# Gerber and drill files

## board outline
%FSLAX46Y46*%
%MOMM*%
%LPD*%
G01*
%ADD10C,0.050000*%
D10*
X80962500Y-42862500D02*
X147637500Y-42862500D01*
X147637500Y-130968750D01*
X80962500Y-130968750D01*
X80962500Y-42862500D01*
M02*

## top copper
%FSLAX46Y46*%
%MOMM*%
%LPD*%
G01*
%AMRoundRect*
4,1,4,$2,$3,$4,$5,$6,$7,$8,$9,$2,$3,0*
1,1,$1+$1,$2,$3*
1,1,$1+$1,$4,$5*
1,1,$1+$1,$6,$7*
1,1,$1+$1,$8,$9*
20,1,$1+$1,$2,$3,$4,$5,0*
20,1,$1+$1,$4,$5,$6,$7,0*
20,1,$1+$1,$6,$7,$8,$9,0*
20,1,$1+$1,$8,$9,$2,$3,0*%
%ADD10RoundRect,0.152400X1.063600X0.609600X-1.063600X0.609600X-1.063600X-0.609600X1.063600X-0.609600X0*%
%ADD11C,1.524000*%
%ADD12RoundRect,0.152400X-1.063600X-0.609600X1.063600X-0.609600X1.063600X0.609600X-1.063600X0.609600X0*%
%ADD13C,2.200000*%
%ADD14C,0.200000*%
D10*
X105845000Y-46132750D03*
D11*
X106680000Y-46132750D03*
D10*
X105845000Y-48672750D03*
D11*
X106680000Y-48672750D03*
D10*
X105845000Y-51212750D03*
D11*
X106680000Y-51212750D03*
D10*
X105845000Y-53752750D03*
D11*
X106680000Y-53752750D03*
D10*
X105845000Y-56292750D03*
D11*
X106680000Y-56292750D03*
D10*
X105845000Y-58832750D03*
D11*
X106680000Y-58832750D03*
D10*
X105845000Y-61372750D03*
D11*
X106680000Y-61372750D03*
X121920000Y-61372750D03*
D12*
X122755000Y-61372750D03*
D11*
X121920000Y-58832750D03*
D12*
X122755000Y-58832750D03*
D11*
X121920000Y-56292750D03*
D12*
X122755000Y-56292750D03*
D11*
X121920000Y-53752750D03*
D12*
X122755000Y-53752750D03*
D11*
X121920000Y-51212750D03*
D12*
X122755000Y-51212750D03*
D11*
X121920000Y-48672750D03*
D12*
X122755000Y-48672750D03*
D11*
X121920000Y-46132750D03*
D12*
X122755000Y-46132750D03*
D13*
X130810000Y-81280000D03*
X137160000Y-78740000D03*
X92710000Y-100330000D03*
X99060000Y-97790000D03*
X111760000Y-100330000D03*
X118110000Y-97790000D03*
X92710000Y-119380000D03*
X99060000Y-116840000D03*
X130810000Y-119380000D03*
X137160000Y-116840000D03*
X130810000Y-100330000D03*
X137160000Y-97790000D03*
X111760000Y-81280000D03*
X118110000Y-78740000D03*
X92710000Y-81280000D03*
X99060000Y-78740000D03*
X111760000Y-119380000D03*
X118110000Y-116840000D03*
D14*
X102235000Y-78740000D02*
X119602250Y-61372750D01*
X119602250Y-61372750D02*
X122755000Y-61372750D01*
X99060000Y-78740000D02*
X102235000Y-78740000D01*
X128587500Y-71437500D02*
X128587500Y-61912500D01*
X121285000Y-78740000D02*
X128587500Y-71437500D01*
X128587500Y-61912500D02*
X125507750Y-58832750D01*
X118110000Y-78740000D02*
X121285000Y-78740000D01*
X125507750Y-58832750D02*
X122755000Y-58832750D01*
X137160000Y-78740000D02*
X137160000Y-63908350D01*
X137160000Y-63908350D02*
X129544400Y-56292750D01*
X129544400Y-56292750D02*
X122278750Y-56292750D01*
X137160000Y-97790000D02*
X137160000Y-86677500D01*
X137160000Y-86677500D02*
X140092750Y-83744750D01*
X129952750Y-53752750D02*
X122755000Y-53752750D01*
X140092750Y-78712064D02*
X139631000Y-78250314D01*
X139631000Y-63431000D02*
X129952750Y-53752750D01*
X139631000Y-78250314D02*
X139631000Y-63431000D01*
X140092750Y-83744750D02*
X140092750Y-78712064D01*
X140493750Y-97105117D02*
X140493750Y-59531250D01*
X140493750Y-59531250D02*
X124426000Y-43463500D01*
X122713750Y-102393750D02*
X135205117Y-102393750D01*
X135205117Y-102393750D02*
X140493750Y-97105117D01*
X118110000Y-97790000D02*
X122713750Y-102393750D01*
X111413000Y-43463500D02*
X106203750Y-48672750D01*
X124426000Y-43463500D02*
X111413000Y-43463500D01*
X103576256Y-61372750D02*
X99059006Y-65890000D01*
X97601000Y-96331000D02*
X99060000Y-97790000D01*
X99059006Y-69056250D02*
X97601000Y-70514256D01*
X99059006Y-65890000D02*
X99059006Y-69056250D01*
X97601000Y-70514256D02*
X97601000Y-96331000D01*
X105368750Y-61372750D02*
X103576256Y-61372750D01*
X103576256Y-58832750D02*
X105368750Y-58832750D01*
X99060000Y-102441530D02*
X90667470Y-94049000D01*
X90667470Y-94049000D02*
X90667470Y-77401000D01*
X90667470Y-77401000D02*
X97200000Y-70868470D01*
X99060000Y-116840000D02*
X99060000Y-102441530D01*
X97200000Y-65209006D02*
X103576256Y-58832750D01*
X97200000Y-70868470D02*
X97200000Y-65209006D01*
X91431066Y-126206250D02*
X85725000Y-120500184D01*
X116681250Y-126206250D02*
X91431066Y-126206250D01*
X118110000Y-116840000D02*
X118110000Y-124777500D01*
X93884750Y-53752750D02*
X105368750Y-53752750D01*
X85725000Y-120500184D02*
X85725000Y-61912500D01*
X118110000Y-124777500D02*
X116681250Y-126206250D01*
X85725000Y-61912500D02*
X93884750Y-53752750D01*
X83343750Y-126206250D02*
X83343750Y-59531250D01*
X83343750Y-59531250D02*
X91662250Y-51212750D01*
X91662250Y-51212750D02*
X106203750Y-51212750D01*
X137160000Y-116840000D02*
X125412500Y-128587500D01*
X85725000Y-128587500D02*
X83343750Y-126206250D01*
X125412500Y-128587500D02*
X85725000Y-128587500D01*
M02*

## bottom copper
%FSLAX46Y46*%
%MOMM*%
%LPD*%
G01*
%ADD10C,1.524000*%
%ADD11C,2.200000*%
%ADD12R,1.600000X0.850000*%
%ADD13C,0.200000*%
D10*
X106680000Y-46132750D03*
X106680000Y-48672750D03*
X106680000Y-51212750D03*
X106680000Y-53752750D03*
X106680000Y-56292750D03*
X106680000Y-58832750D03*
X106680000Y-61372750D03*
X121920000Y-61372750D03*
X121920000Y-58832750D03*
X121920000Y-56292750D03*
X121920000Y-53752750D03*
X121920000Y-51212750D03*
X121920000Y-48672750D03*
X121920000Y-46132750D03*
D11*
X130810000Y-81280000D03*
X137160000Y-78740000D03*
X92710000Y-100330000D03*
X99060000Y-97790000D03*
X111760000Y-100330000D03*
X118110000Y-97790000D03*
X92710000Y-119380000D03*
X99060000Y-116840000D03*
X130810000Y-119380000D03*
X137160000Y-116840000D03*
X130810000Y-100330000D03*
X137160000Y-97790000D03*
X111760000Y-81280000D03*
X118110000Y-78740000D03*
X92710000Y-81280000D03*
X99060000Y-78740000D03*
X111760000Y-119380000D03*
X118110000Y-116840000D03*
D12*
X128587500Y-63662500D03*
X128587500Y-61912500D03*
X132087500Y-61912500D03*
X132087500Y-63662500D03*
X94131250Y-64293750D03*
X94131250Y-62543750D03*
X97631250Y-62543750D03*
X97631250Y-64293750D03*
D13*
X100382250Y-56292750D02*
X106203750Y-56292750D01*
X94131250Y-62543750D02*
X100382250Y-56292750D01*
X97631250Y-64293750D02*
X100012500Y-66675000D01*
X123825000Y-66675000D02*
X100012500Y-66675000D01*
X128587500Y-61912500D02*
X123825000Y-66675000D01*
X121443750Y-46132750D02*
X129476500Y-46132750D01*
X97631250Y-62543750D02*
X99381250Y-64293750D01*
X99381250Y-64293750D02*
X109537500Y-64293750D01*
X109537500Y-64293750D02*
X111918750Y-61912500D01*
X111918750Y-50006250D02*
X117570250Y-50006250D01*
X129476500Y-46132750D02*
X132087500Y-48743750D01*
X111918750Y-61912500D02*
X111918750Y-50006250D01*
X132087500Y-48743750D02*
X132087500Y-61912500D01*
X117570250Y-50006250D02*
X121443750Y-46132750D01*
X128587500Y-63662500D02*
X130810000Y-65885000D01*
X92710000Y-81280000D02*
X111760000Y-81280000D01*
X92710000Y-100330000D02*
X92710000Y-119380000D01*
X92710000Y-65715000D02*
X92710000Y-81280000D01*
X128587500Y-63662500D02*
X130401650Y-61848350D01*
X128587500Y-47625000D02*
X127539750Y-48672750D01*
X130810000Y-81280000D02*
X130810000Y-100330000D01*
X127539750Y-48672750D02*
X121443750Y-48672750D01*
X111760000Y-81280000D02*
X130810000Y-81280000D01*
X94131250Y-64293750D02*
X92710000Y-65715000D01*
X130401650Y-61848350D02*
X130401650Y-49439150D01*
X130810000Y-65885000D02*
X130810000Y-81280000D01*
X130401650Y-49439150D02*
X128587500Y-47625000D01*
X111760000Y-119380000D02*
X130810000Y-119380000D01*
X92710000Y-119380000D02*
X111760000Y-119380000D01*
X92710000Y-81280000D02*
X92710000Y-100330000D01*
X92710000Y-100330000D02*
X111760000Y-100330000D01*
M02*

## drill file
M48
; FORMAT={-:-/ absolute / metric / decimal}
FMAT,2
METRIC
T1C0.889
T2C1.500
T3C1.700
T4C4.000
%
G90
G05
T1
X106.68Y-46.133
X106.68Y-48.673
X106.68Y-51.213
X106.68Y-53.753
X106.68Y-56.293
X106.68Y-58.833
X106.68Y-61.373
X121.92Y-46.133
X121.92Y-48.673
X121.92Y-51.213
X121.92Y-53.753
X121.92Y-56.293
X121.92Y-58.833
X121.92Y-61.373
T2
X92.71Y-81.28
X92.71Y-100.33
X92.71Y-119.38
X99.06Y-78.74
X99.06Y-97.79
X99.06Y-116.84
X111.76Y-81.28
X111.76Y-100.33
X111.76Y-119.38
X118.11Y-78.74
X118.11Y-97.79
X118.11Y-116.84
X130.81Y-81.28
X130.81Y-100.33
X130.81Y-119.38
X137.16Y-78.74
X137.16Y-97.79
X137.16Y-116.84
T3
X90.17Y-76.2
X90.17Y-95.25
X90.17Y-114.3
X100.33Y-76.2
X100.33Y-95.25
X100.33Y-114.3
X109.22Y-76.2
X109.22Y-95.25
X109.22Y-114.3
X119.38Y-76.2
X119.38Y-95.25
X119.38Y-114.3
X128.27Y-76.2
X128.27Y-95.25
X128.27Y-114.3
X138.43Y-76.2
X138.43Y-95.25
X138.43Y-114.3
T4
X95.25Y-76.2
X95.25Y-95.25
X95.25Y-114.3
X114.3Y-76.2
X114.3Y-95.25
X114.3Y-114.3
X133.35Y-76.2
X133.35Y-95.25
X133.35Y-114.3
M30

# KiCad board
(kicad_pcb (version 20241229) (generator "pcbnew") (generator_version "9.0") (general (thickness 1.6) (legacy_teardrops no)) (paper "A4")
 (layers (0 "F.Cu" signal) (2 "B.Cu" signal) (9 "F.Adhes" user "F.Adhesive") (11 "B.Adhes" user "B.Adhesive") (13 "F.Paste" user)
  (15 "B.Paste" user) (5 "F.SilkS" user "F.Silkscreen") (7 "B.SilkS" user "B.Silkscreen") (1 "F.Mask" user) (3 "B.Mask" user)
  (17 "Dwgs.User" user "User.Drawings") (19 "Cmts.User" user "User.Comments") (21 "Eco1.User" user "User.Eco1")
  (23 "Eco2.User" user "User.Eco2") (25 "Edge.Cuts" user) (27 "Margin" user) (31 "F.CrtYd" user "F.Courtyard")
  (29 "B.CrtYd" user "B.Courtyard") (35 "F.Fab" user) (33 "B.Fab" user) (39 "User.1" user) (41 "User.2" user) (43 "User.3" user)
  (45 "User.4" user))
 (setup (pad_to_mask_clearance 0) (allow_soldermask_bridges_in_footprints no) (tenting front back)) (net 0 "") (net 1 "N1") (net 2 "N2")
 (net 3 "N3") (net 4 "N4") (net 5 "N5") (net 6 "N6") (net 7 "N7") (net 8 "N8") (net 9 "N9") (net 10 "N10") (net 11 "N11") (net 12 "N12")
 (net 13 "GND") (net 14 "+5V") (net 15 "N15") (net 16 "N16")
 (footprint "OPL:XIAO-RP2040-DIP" (layer "F.Cu") (at 114.3 53.75275)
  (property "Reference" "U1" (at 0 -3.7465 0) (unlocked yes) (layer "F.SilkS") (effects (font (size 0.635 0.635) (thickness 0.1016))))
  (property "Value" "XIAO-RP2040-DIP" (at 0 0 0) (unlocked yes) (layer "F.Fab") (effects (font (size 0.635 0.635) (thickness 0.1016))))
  (pad "1" smd roundrect (at -8.455 -7.62 180) (size 2.432 1.524) (layers "F.Cu" "F.Mask") (roundrect_rratio 0.1) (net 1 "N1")
   (thermal_bridge_angle 45))
  (pad "1" thru_hole circle (at -7.62 -7.62 180) (size 1.524 1.524) (drill 0.889) (layers "*.Cu" "*.Mask") (remove_unused_layers no)
   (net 1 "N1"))
  (pad "2" smd roundrect (at -8.455 -5.08 180) (size 2.432 1.524) (layers "F.Cu" "F.Mask") (roundrect_rratio 0.1) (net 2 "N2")
   (thermal_bridge_angle 45))
  (pad "2" thru_hole circle (at -7.62 -5.08 180) (size 1.524 1.524) (drill 0.889) (layers "*.Cu" "*.Mask") (remove_unused_layers no)
   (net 2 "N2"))
  (pad "3" smd roundrect (at -8.455 -2.54 180) (size 2.432 1.524) (layers "F.Cu" "F.Mask") (roundrect_rratio 0.1) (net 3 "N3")
   (thermal_bridge_angle 45))
  (pad "3" thru_hole circle (at -7.62 -2.54 180) (size 1.524 1.524) (drill 0.889) (layers "*.Cu" "*.Mask") (remove_unused_layers no)
   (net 3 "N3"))
  (pad "4" smd roundrect (at -8.455 0 180) (size 2.432 1.524) (layers "F.Cu" "F.Mask") (roundrect_rratio 0.1) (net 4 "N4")
   (thermal_bridge_angle 45))
  (pad "4" thru_hole circle (at -7.62 0 180) (size 1.524 1.524) (drill 0.889) (layers "*.Cu" "*.Mask") (remove_unused_layers no)
   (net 4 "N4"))
  (pad "5" smd roundrect (at -8.455 2.54 180) (size 2.432 1.524) (layers "F.Cu" "F.Mask") (roundrect_rratio 0.1) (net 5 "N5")
   (thermal_bridge_angle 45))
  (pad "5" thru_hole circle (at -7.62 2.54 180) (size 1.524 1.524) (drill 0.889) (layers "*.Cu" "*.Mask") (remove_unused_layers no)
   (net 5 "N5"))
  (pad "6" smd roundrect (at -8.455 5.08 180) (size 2.432 1.524) (layers "F.Cu" "F.Mask") (roundrect_rratio 0.1) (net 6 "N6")
   (thermal_bridge_angle 45))
  (pad "6" thru_hole circle (at -7.62 5.08 180) (size 1.524 1.524) (drill 0.889) (layers "*.Cu" "*.Mask") (remove_unused_layers no)
   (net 6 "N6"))
  (pad "7" smd roundrect (at -8.455 7.62 180) (size 2.432 1.524) (layers "F.Cu" "F.Mask") (roundrect_rratio 0.1) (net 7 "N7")
   (thermal_bridge_angle 45))
  (pad "7" thru_hole circle (at -7.62 7.62 180) (size 1.524 1.524) (drill 0.889) (layers "*.Cu" "*.Mask") (remove_unused_layers no)
   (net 7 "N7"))
  (pad "8" thru_hole circle (at 7.62 7.62) (size 1.524 1.524) (drill 0.889) (layers "*.Cu" "*.Mask") (remove_unused_layers no) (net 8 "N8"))
  (pad "8" smd roundrect (at 8.455 7.62) (size 2.432 1.524) (layers "F.Cu" "F.Mask") (roundrect_rratio 0.1) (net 8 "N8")
   (thermal_bridge_angle 45))
  (pad "9" thru_hole circle (at 7.62 5.08) (size 1.524 1.524) (drill 0.889) (layers "*.Cu" "*.Mask") (remove_unused_layers no) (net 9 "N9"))
  (pad "9" smd roundrect (at 8.455 5.08) (size 2.432 1.524) (layers "F.Cu" "F.Mask") (roundrect_rratio 0.1) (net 9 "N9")
   (thermal_bridge_angle 45))
  (pad "10" thru_hole circle (at 7.62 2.54) (size 1.524 1.524) (drill 0.889) (layers "*.Cu" "*.Mask") (remove_unused_layers no)
   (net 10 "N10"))
  (pad "10" smd roundrect (at 8.455 2.54) (size 2.432 1.524) (layers "F.Cu" "F.Mask") (roundrect_rratio 0.1) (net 10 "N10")
   (thermal_bridge_angle 45))
  (pad "11" thru_hole circle (at 7.62 0) (size 1.524 1.524) (drill 0.889) (layers "*.Cu" "*.Mask") (remove_unused_layers no) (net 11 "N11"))
  (pad "11" smd roundrect (at 8.455 0) (size 2.432 1.524) (layers "F.Cu" "F.Mask") (roundrect_rratio 0.1) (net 11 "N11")
   (thermal_bridge_angle 45))
  (pad "12" thru_hole circle (at 7.62 -2.54) (size 1.524 1.524) (drill 0.889) (layers "*.Cu" "*.Mask") (remove_unused_layers no)
   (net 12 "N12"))
  (pad "12" smd roundrect (at 8.455 -2.54) (size 2.432 1.524) (layers "F.Cu" "F.Mask") (roundrect_rratio 0.1) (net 12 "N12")
   (thermal_bridge_angle 45))
  (pad "13" thru_hole circle (at 7.62 -5.08) (size 1.524 1.524) (drill 0.889) (layers "*.Cu" "*.Mask") (remove_unused_layers no)
   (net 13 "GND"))
  (pad "13" smd roundrect (at 8.455 -5.08) (size 2.432 1.524) (layers "F.Cu" "F.Mask") (roundrect_rratio 0.1) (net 13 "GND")
   (thermal_bridge_angle 45))
  (pad "14" thru_hole circle (at 7.62 -7.62) (size 1.524 1.524) (drill 0.889) (layers "*.Cu" "*.Mask") (remove_unused_layers no)
   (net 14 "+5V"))
  (pad "14" smd roundrect (at 8.455 -7.62) (size 2.432 1.524) (layers "F.Cu" "F.Mask") (roundrect_rratio 0.1) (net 14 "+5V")
   (thermal_bridge_angle 45)))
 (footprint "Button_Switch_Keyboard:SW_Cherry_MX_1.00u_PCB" (layer "F.Cu") (at 130.81 81.28 180)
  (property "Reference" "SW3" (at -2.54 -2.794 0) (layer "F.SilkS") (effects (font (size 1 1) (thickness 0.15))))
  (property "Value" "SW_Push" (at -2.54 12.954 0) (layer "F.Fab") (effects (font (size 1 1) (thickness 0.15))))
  (pad "" np_thru_hole circle (at -7.62 5.08 180) (size 1.7 1.7) (drill 1.7) (layers "*.Cu" "*.Mask"))
  (pad "" np_thru_hole circle (at -2.54 5.08 180) (size 4 4) (drill 4) (layers "*.Cu" "*.Mask"))
  (pad "" np_thru_hole circle (at 2.54 5.08 180) (size 1.7 1.7) (drill 1.7) (layers "*.Cu" "*.Mask"))
  (pad "1" thru_hole circle (at 0 0 180) (size 2.2 2.2) (drill 1.5) (layers "*.Cu" "*.Mask") (remove_unused_layers no) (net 13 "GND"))
  (pad "2" thru_hole circle (at -6.35 2.54 180) (size 2.2 2.2) (drill 1.5) (layers "*.Cu" "*.Mask") (remove_unused_layers no) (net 10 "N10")))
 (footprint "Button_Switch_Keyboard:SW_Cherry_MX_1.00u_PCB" (layer "F.Cu") (at 92.71 100.33 180)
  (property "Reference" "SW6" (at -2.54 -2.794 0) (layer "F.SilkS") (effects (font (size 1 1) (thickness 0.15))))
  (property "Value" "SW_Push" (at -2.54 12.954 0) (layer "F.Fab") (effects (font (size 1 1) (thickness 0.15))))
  (pad "" np_thru_hole circle (at -7.62 5.08 180) (size 1.7 1.7) (drill 1.7) (layers "*.Cu" "*.Mask"))
  (pad "" np_thru_hole circle (at -2.54 5.08 180) (size 4 4) (drill 4) (layers "*.Cu" "*.Mask"))
  (pad "" np_thru_hole circle (at 2.54 5.08 180) (size 1.7 1.7) (drill 1.7) (layers "*.Cu" "*.Mask"))
  (pad "1" thru_hole circle (at 0 0 180) (size 2.2 2.2) (drill 1.5) (layers "*.Cu" "*.Mask") (remove_unused_layers no) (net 13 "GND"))
  (pad "2" thru_hole circle (at -6.35 2.54 180) (size 2.2 2.2) (drill 1.5) (layers "*.Cu" "*.Mask") (remove_unused_layers no) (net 7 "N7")))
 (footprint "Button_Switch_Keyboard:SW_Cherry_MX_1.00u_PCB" (layer "F.Cu") (at 111.76 100.33 180)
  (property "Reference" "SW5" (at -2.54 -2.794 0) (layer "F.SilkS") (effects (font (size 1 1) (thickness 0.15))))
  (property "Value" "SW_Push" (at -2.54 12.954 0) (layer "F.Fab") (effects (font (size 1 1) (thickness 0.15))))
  (pad "" np_thru_hole circle (at -7.62 5.08 180) (size 1.7 1.7) (drill 1.7) (layers "*.Cu" "*.Mask"))
  (pad "" np_thru_hole circle (at -2.54 5.08 180) (size 4 4) (drill 4) (layers "*.Cu" "*.Mask"))
  (pad "" np_thru_hole circle (at 2.54 5.08 180) (size 1.7 1.7) (drill 1.7) (layers "*.Cu" "*.Mask"))
  (pad "1" thru_hole circle (at 0 0 180) (size 2.2 2.2) (drill 1.5) (layers "*.Cu" "*.Mask") (remove_unused_layers no) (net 13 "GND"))
  (pad "2" thru_hole circle (at -6.35 2.54 180) (size 2.2 2.2) (drill 1.5) (layers "*.Cu" "*.Mask") (remove_unused_layers no) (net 2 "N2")))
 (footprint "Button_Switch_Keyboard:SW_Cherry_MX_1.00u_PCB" (layer "F.Cu") (at 92.71 119.38 180)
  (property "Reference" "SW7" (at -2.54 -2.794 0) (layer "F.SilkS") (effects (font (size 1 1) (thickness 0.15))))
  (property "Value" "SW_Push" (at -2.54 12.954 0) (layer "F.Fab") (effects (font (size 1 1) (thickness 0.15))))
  (pad "" np_thru_hole circle (at -7.62 5.08 180) (size 1.7 1.7) (drill 1.7) (layers "*.Cu" "*.Mask"))
  (pad "" np_thru_hole circle (at -2.54 5.08 180) (size 4 4) (drill 4) (layers "*.Cu" "*.Mask"))
  (pad "" np_thru_hole circle (at 2.54 5.08 180) (size 1.7 1.7) (drill 1.7) (layers "*.Cu" "*.Mask"))
  (pad "1" thru_hole circle (at 0 0 180) (size 2.2 2.2) (drill 1.5) (layers "*.Cu" "*.Mask") (remove_unused_layers no) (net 13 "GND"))
  (pad "2" thru_hole circle (at -6.35 2.54 180) (size 2.2 2.2) (drill 1.5) (layers "*.Cu" "*.Mask") (remove_unused_layers no) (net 6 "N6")))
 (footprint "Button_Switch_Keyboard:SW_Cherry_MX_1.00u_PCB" (layer "F.Cu") (at 130.81 119.38 180)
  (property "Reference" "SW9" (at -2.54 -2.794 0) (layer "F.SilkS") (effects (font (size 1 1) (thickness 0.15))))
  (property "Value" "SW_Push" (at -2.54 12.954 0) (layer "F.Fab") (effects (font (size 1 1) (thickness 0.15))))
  (pad "" np_thru_hole circle (at -7.62 5.08 180) (size 1.7 1.7) (drill 1.7) (layers "*.Cu" "*.Mask"))
  (pad "" np_thru_hole circle (at -2.54 5.08 180) (size 4 4) (drill 4) (layers "*.Cu" "*.Mask"))
  (pad "" np_thru_hole circle (at 2.54 5.08 180) (size 1.7 1.7) (drill 1.7) (layers "*.Cu" "*.Mask"))
  (pad "1" thru_hole circle (at 0 0 180) (size 2.2 2.2) (drill 1.5) (layers "*.Cu" "*.Mask") (remove_unused_layers no) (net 13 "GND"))
  (pad "2" thru_hole circle (at -6.35 2.54 180) (size 2.2 2.2) (drill 1.5) (layers "*.Cu" "*.Mask") (remove_unused_layers no) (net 3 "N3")))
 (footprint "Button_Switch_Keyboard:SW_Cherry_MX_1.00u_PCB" (layer "F.Cu") (at 130.81 100.33 180)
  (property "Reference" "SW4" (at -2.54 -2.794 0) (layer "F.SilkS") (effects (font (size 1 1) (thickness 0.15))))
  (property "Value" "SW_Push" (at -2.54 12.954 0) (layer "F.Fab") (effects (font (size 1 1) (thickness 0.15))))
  (pad "" np_thru_hole circle (at -7.62 5.08 180) (size 1.7 1.7) (drill 1.7) (layers "*.Cu" "*.Mask"))
  (pad "" np_thru_hole circle (at -2.54 5.08 180) (size 4 4) (drill 4) (layers "*.Cu" "*.Mask"))
  (pad "" np_thru_hole circle (at 2.54 5.08 180) (size 1.7 1.7) (drill 1.7) (layers "*.Cu" "*.Mask"))
  (pad "1" thru_hole circle (at 0 0 180) (size 2.2 2.2) (drill 1.5) (layers "*.Cu" "*.Mask") (remove_unused_layers no) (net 13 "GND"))
  (pad "2" thru_hole circle (at -6.35 2.54 180) (size 2.2 2.2) (drill 1.5) (layers "*.Cu" "*.Mask") (remove_unused_layers no) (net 11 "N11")))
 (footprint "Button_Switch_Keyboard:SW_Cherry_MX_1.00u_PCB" (layer "F.Cu") (at 111.76 81.28 180)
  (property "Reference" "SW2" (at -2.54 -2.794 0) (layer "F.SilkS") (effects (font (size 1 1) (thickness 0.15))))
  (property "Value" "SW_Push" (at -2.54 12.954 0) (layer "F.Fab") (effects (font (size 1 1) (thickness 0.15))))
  (pad "" np_thru_hole circle (at -7.62 5.08 180) (size 1.7 1.7) (drill 1.7) (layers "*.Cu" "*.Mask"))
  (pad "" np_thru_hole circle (at -2.54 5.08 180) (size 4 4) (drill 4) (layers "*.Cu" "*.Mask"))
  (pad "" np_thru_hole circle (at 2.54 5.08 180) (size 1.7 1.7) (drill 1.7) (layers "*.Cu" "*.Mask"))
  (pad "1" thru_hole circle (at 0 0 180) (size 2.2 2.2) (drill 1.5) (layers "*.Cu" "*.Mask") (remove_unused_layers no) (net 13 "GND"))
  (pad "2" thru_hole circle (at -6.35 2.54 180) (size 2.2 2.2) (drill 1.5) (layers "*.Cu" "*.Mask") (remove_unused_layers no) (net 9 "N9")))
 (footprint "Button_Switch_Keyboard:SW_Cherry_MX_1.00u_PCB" (layer "F.Cu") (at 92.71 81.28 180)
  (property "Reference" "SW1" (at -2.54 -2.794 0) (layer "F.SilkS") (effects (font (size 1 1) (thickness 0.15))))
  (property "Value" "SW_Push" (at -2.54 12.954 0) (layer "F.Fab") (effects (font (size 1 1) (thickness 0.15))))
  (pad "" np_thru_hole circle (at -7.62 5.08 180) (size 1.7 1.7) (drill 1.7) (layers "*.Cu" "*.Mask"))
  (pad "" np_thru_hole circle (at -2.54 5.08 180) (size 4 4) (drill 4) (layers "*.Cu" "*.Mask"))
  (pad "" np_thru_hole circle (at 2.54 5.08 180) (size 1.7 1.7) (drill 1.7) (layers "*.Cu" "*.Mask"))
  (pad "1" thru_hole circle (at 0 0 180) (size 2.2 2.2) (drill 1.5) (layers "*.Cu" "*.Mask") (remove_unused_layers no) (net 13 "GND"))
  (pad "2" thru_hole circle (at -6.35 2.54 180) (size 2.2 2.2) (drill 1.5) (layers "*.Cu" "*.Mask") (remove_unused_layers no) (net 8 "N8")))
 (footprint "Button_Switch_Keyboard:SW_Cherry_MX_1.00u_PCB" (layer "F.Cu") (at 111.76 119.38 180)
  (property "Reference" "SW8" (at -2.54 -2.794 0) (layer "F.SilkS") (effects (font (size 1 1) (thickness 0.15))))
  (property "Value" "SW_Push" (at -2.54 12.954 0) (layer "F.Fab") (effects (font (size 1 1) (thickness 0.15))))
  (pad "" np_thru_hole circle (at -7.62 5.08 180) (size 1.7 1.7) (drill 1.7) (layers "*.Cu" "*.Mask"))
  (pad "" np_thru_hole circle (at -2.54 5.08 180) (size 4 4) (drill 4) (layers "*.Cu" "*.Mask"))
  (pad "" np_thru_hole circle (at 2.54 5.08 180) (size 1.7 1.7) (drill 1.7) (layers "*.Cu" "*.Mask"))
  (pad "1" thru_hole circle (at 0 0 180) (size 2.2 2.2) (drill 1.5) (layers "*.Cu" "*.Mask") (remove_unused_layers no) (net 13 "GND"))
  (pad "2" thru_hole circle (at -6.35 2.54 180) (size 2.2 2.2) (drill 1.5) (layers "*.Cu" "*.Mask") (remove_unused_layers no) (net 4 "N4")))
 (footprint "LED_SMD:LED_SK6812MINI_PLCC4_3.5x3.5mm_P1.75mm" (layer "B.Cu") (at 130.3375 62.7875)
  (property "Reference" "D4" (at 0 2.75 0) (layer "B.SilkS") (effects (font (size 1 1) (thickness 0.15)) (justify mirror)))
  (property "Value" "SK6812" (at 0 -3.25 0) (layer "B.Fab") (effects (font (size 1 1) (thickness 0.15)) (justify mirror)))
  (pad "1" smd rect (at -1.75 0.875) (size 1.6 0.85) (layers "B.Cu" "B.Mask" "B.Paste") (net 13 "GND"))
  (pad "2" smd rect (at -1.75 -0.875) (size 1.6 0.85) (layers "B.Cu" "B.Mask" "B.Paste") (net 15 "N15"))
  (pad "3" smd rect (at 1.75 -0.875) (size 1.6 0.85) (layers "B.Cu" "B.Mask" "B.Paste") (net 14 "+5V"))
  (pad "4" smd rect (at 1.75 0.875) (size 1.6 0.85) (layers "B.Cu" "B.Mask" "B.Paste") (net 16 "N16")))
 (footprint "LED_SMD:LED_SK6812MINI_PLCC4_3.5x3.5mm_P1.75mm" (layer "B.Cu") (at 95.88125 63.41875)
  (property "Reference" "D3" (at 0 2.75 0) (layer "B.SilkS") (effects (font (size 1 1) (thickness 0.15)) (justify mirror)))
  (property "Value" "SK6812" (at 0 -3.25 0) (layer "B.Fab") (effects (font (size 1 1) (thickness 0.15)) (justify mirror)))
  (pad "1" smd rect (at -1.75 0.875) (size 1.6 0.85) (layers "B.Cu" "B.Mask" "B.Paste") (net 13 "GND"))
  (pad "2" smd rect (at -1.75 -0.875) (size 1.6 0.85) (layers "B.Cu" "B.Mask" "B.Paste") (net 5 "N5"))
  (pad "3" smd rect (at 1.75 -0.875) (size 1.6 0.85) (layers "B.Cu" "B.Mask" "B.Paste") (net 14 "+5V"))
  (pad "4" smd rect (at 1.75 0.875) (size 1.6 0.85) (layers "B.Cu" "B.Mask" "B.Paste") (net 15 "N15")))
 (gr_rect (start 80.9625 42.8625) (end 147.6375 130.96875) (stroke (width 0.05) (type solid)) (fill no) (layer "Edge.Cuts"))
 (segment (start 100.38225 56.29275) (end 106.20375 56.29275) (width 0.2) (layer "B.Cu") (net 5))
 (segment (start 94.13125 62.54375) (end 100.38225 56.29275) (width 0.2) (layer "B.Cu") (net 5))
 (segment (start 97.63125 64.29375) (end 100.0125 66.675) (width 0.2) (layer "B.Cu") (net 15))
 (segment (start 123.825 66.675) (end 100.0125 66.675) (width 0.2) (layer "B.Cu") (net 15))
 (segment (start 128.5875 61.9125) (end 123.825 66.675) (width 0.2) (layer "B.Cu") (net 15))
 (segment (start 121.44375 46.13275) (end 129.4765 46.13275) (width 0.2) (layer "B.Cu") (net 14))
 (segment (start 97.63125 62.54375) (end 99.38125 64.29375) (width 0.2) (layer "B.Cu") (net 14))
 (segment (start 99.38125 64.29375) (end 109.5375 64.29375) (width 0.2) (layer "B.Cu") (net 14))
 (segment (start 109.5375 64.29375) (end 111.91875 61.9125) (width 0.2) (layer "B.Cu") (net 14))
 (segment (start 111.91875 50.00625) (end 117.57025 50.00625) (width 0.2) (layer "B.Cu") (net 14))
 (segment (start 129.4765 46.13275) (end 132.0875 48.74375) (width 0.2) (layer "B.Cu") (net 14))
 (segment (start 111.91875 61.9125) (end 111.91875 50.00625) (width 0.2) (layer "B.Cu") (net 14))
 (segment (start 132.0875 48.74375) (end 132.0875 61.9125) (width 0.2) (layer "B.Cu") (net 14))
 (segment (start 117.57025 50.00625) (end 121.44375 46.13275) (width 0.2) (layer "B.Cu") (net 14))
 (segment (start 128.5875 63.6625) (end 130.81 65.885) (width 0.2) (layer "B.Cu") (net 13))
 (segment (start 92.71 81.28) (end 111.76 81.28) (width 0.2) (layer "B.Cu") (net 13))
 (segment (start 92.71 100.33) (end 92.71 119.38) (width 0.2) (layer "B.Cu") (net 13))
 (segment (start 92.71 65.715) (end 92.71 81.28) (width 0.2) (layer "B.Cu") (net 13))
 (segment (start 128.5875 63.6625) (end 130.40165 61.84835) (width 0.2) (layer "B.Cu") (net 13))
 (segment (start 128.5875 47.625) (end 127.53975 48.67275) (width 0.2) (layer "B.Cu") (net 13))
 (segment (start 130.81 81.28) (end 130.81 100.33) (width 0.2) (layer "B.Cu") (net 13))
 (segment (start 127.53975 48.67275) (end 121.44375 48.67275) (width 0.2) (layer "B.Cu") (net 13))
 (segment (start 111.76 81.28) (end 130.81 81.28) (width 0.2) (layer "B.Cu") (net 13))
 (segment (start 94.13125 64.29375) (end 92.71 65.715) (width 0.2) (layer "B.Cu") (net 13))
 (segment (start 130.40165 61.84835) (end 130.40165 49.43915) (width 0.2) (layer "B.Cu") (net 13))
 (segment (start 130.81 65.885) (end 130.81 81.28) (width 0.2) (layer "B.Cu") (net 13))
 (segment (start 130.40165 49.43915) (end 128.5875 47.625) (width 0.2) (layer "B.Cu") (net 13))
 (segment (start 111.76 119.38) (end 130.81 119.38) (width 0.2) (layer "B.Cu") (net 13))
 (segment (start 92.71 119.38) (end 111.76 119.38) (width 0.2) (layer "B.Cu") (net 13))
 (segment (start 92.71 81.28) (end 92.71 100.33) (width 0.2) (layer "B.Cu") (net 13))
 (segment (start 92.71 100.33) (end 111.76 100.33) (width 0.2) (layer "B.Cu") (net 13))
 (segment (start 102.235 78.74) (end 119.60225 61.37275) (width 0.2) (layer "F.Cu") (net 8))
 (segment (start 119.60225 61.37275) (end 122.755 61.37275) (width 0.2) (layer "F.Cu") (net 8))
 (segment (start 99.06 78.74) (end 102.235 78.74) (width 0.2) (layer "F.Cu") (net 8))
 (segment (start 128.5875 71.4375) (end 128.5875 61.9125) (width 0.2) (layer "F.Cu") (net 9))
 (segment (start 121.285 78.74) (end 128.5875 71.4375) (width 0.2) (layer "F.Cu") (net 9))
 (segment (start 128.5875 61.9125) (end 125.50775 58.83275) (width 0.2) (layer "F.Cu") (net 9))
 (segment (start 118.11 78.74) (end 121.285 78.74) (width 0.2) (layer "F.Cu") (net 9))
 (segment (start 125.50775 58.83275) (end 122.755 58.83275) (width 0.2) (layer "F.Cu") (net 9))
 (segment (start 137.16 78.74) (end 137.16 63.90835) (width 0.2) (layer "F.Cu") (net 10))
 (segment (start 137.16 63.90835) (end 129.5444 56.29275) (width 0.2) (layer "F.Cu") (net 10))
 (segment (start 129.5444 56.29275) (end 122.27875 56.29275) (width 0.2) (layer "F.Cu") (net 10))
 (segment (start 137.16 97.79) (end 137.16 86.6775) (width 0.2) (layer "F.Cu") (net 11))
 (segment (start 137.16 86.6775) (end 140.09275 83.74475) (width 0.2) (layer "F.Cu") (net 11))
 (segment (start 129.95275 53.75275) (end 122.755 53.75275) (width 0.2) (layer "F.Cu") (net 11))
 (segment (start 140.09275 78.712064) (end 139.631 78.250314) (width 0.2) (layer "F.Cu") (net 11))
 (segment (start 139.631 63.431) (end 129.95275 53.75275) (width 0.2) (layer "F.Cu") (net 11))
 (segment (start 139.631 78.250314) (end 139.631 63.431) (width 0.2) (layer "F.Cu") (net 11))
 (segment (start 140.09275 83.74475) (end 140.09275 78.712064) (width 0.2) (layer "F.Cu") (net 11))
 (segment (start 140.49375 97.105117) (end 140.49375 59.53125) (width 0.2) (layer "F.Cu") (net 2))
 (segment (start 140.49375 59.53125) (end 124.426 43.4635) (width 0.2) (layer "F.Cu") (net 2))
 (segment (start 122.71375 102.39375) (end 135.205117 102.39375) (width 0.2) (layer "F.Cu") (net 2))
 (segment (start 135.205117 102.39375) (end 140.49375 97.105117) (width 0.2) (layer "F.Cu") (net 2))
 (segment (start 118.11 97.79) (end 122.71375 102.39375) (width 0.2) (layer "F.Cu") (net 2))
 (segment (start 111.413 43.4635) (end 106.20375 48.67275) (width 0.2) (layer "F.Cu") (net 2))
 (segment (start 124.426 43.4635) (end 111.413 43.4635) (width 0.2) (layer "F.Cu") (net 2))
 (segment (start 103.576256 61.37275) (end 99.059006 65.89) (width 0.2) (layer "F.Cu") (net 7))
 (segment (start 97.601 96.331) (end 99.06 97.79) (width 0.2) (layer "F.Cu") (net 7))
 (segment (start 99.059006 69.05625) (end 97.601 70.514256) (width 0.2) (layer "F.Cu") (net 7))
 (segment (start 99.059006 65.89) (end 99.059006 69.05625) (width 0.2) (layer "F.Cu") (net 7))
 (segment (start 97.601 70.514256) (end 97.601 96.331) (width 0.2) (layer "F.Cu") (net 7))
 (segment (start 105.36875 61.37275) (end 103.576256 61.37275) (width 0.2) (layer "F.Cu") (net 7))
 (segment (start 103.576256 58.83275) (end 105.36875 58.83275) (width 0.2) (layer "F.Cu") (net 6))
 (segment (start 99.06 102.44153) (end 90.66747 94.049) (width 0.2) (layer "F.Cu") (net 6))
 (segment (start 90.66747 94.049) (end 90.66747 77.401) (width 0.2) (layer "F.Cu") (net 6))
 (segment (start 90.66747 77.401) (end 97.2 70.86847) (width 0.2) (layer "F.Cu") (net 6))
 (segment (start 99.06 116.84) (end 99.06 102.44153) (width 0.2) (layer "F.Cu") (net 6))
 (segment (start 97.2 65.209006) (end 103.576256 58.83275) (width 0.2) (layer "F.Cu") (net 6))
 (segment (start 97.2 70.86847) (end 97.2 65.209006) (width 0.2) (layer "F.Cu") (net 6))
 (segment (start 91.431066 126.20625) (end 85.725 120.500184) (width 0.2) (layer "F.Cu") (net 4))
 (segment (start 116.68125 126.20625) (end 91.431066 126.20625) (width 0.2) (layer "F.Cu") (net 4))
 (segment (start 118.11 116.84) (end 118.11 124.7775) (width 0.2) (layer "F.Cu") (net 4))
 (segment (start 93.88475 53.75275) (end 105.36875 53.75275) (width 0.2) (layer "F.Cu") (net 4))
 (segment (start 85.725 120.500184) (end 85.725 61.9125) (width 0.2) (layer "F.Cu") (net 4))
 (segment (start 118.11 124.7775) (end 116.68125 126.20625) (width 0.2) (layer "F.Cu") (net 4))
 (segment (start 85.725 61.9125) (end 93.88475 53.75275) (width 0.2) (layer "F.Cu") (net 4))
 (segment (start 83.34375 126.20625) (end 83.34375 59.53125) (width 0.2) (layer "F.Cu") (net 3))
 (segment (start 83.34375 59.53125) (end 91.66225 51.21275) (width 0.2) (layer "F.Cu") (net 3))
 (segment (start 91.66225 51.21275) (end 106.20375 51.21275) (width 0.2) (layer "F.Cu") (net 3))
 (segment (start 137.16 116.84) (end 125.4125 128.5875) (width 0.2) (layer "F.Cu") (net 3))
 (segment (start 85.725 128.5875) (end 83.34375 126.20625) (width 0.2) (layer "F.Cu") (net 3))
 (segment (start 125.4125 128.5875) (end 85.725 128.5875) (width 0.2) (layer "F.Cu") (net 3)))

